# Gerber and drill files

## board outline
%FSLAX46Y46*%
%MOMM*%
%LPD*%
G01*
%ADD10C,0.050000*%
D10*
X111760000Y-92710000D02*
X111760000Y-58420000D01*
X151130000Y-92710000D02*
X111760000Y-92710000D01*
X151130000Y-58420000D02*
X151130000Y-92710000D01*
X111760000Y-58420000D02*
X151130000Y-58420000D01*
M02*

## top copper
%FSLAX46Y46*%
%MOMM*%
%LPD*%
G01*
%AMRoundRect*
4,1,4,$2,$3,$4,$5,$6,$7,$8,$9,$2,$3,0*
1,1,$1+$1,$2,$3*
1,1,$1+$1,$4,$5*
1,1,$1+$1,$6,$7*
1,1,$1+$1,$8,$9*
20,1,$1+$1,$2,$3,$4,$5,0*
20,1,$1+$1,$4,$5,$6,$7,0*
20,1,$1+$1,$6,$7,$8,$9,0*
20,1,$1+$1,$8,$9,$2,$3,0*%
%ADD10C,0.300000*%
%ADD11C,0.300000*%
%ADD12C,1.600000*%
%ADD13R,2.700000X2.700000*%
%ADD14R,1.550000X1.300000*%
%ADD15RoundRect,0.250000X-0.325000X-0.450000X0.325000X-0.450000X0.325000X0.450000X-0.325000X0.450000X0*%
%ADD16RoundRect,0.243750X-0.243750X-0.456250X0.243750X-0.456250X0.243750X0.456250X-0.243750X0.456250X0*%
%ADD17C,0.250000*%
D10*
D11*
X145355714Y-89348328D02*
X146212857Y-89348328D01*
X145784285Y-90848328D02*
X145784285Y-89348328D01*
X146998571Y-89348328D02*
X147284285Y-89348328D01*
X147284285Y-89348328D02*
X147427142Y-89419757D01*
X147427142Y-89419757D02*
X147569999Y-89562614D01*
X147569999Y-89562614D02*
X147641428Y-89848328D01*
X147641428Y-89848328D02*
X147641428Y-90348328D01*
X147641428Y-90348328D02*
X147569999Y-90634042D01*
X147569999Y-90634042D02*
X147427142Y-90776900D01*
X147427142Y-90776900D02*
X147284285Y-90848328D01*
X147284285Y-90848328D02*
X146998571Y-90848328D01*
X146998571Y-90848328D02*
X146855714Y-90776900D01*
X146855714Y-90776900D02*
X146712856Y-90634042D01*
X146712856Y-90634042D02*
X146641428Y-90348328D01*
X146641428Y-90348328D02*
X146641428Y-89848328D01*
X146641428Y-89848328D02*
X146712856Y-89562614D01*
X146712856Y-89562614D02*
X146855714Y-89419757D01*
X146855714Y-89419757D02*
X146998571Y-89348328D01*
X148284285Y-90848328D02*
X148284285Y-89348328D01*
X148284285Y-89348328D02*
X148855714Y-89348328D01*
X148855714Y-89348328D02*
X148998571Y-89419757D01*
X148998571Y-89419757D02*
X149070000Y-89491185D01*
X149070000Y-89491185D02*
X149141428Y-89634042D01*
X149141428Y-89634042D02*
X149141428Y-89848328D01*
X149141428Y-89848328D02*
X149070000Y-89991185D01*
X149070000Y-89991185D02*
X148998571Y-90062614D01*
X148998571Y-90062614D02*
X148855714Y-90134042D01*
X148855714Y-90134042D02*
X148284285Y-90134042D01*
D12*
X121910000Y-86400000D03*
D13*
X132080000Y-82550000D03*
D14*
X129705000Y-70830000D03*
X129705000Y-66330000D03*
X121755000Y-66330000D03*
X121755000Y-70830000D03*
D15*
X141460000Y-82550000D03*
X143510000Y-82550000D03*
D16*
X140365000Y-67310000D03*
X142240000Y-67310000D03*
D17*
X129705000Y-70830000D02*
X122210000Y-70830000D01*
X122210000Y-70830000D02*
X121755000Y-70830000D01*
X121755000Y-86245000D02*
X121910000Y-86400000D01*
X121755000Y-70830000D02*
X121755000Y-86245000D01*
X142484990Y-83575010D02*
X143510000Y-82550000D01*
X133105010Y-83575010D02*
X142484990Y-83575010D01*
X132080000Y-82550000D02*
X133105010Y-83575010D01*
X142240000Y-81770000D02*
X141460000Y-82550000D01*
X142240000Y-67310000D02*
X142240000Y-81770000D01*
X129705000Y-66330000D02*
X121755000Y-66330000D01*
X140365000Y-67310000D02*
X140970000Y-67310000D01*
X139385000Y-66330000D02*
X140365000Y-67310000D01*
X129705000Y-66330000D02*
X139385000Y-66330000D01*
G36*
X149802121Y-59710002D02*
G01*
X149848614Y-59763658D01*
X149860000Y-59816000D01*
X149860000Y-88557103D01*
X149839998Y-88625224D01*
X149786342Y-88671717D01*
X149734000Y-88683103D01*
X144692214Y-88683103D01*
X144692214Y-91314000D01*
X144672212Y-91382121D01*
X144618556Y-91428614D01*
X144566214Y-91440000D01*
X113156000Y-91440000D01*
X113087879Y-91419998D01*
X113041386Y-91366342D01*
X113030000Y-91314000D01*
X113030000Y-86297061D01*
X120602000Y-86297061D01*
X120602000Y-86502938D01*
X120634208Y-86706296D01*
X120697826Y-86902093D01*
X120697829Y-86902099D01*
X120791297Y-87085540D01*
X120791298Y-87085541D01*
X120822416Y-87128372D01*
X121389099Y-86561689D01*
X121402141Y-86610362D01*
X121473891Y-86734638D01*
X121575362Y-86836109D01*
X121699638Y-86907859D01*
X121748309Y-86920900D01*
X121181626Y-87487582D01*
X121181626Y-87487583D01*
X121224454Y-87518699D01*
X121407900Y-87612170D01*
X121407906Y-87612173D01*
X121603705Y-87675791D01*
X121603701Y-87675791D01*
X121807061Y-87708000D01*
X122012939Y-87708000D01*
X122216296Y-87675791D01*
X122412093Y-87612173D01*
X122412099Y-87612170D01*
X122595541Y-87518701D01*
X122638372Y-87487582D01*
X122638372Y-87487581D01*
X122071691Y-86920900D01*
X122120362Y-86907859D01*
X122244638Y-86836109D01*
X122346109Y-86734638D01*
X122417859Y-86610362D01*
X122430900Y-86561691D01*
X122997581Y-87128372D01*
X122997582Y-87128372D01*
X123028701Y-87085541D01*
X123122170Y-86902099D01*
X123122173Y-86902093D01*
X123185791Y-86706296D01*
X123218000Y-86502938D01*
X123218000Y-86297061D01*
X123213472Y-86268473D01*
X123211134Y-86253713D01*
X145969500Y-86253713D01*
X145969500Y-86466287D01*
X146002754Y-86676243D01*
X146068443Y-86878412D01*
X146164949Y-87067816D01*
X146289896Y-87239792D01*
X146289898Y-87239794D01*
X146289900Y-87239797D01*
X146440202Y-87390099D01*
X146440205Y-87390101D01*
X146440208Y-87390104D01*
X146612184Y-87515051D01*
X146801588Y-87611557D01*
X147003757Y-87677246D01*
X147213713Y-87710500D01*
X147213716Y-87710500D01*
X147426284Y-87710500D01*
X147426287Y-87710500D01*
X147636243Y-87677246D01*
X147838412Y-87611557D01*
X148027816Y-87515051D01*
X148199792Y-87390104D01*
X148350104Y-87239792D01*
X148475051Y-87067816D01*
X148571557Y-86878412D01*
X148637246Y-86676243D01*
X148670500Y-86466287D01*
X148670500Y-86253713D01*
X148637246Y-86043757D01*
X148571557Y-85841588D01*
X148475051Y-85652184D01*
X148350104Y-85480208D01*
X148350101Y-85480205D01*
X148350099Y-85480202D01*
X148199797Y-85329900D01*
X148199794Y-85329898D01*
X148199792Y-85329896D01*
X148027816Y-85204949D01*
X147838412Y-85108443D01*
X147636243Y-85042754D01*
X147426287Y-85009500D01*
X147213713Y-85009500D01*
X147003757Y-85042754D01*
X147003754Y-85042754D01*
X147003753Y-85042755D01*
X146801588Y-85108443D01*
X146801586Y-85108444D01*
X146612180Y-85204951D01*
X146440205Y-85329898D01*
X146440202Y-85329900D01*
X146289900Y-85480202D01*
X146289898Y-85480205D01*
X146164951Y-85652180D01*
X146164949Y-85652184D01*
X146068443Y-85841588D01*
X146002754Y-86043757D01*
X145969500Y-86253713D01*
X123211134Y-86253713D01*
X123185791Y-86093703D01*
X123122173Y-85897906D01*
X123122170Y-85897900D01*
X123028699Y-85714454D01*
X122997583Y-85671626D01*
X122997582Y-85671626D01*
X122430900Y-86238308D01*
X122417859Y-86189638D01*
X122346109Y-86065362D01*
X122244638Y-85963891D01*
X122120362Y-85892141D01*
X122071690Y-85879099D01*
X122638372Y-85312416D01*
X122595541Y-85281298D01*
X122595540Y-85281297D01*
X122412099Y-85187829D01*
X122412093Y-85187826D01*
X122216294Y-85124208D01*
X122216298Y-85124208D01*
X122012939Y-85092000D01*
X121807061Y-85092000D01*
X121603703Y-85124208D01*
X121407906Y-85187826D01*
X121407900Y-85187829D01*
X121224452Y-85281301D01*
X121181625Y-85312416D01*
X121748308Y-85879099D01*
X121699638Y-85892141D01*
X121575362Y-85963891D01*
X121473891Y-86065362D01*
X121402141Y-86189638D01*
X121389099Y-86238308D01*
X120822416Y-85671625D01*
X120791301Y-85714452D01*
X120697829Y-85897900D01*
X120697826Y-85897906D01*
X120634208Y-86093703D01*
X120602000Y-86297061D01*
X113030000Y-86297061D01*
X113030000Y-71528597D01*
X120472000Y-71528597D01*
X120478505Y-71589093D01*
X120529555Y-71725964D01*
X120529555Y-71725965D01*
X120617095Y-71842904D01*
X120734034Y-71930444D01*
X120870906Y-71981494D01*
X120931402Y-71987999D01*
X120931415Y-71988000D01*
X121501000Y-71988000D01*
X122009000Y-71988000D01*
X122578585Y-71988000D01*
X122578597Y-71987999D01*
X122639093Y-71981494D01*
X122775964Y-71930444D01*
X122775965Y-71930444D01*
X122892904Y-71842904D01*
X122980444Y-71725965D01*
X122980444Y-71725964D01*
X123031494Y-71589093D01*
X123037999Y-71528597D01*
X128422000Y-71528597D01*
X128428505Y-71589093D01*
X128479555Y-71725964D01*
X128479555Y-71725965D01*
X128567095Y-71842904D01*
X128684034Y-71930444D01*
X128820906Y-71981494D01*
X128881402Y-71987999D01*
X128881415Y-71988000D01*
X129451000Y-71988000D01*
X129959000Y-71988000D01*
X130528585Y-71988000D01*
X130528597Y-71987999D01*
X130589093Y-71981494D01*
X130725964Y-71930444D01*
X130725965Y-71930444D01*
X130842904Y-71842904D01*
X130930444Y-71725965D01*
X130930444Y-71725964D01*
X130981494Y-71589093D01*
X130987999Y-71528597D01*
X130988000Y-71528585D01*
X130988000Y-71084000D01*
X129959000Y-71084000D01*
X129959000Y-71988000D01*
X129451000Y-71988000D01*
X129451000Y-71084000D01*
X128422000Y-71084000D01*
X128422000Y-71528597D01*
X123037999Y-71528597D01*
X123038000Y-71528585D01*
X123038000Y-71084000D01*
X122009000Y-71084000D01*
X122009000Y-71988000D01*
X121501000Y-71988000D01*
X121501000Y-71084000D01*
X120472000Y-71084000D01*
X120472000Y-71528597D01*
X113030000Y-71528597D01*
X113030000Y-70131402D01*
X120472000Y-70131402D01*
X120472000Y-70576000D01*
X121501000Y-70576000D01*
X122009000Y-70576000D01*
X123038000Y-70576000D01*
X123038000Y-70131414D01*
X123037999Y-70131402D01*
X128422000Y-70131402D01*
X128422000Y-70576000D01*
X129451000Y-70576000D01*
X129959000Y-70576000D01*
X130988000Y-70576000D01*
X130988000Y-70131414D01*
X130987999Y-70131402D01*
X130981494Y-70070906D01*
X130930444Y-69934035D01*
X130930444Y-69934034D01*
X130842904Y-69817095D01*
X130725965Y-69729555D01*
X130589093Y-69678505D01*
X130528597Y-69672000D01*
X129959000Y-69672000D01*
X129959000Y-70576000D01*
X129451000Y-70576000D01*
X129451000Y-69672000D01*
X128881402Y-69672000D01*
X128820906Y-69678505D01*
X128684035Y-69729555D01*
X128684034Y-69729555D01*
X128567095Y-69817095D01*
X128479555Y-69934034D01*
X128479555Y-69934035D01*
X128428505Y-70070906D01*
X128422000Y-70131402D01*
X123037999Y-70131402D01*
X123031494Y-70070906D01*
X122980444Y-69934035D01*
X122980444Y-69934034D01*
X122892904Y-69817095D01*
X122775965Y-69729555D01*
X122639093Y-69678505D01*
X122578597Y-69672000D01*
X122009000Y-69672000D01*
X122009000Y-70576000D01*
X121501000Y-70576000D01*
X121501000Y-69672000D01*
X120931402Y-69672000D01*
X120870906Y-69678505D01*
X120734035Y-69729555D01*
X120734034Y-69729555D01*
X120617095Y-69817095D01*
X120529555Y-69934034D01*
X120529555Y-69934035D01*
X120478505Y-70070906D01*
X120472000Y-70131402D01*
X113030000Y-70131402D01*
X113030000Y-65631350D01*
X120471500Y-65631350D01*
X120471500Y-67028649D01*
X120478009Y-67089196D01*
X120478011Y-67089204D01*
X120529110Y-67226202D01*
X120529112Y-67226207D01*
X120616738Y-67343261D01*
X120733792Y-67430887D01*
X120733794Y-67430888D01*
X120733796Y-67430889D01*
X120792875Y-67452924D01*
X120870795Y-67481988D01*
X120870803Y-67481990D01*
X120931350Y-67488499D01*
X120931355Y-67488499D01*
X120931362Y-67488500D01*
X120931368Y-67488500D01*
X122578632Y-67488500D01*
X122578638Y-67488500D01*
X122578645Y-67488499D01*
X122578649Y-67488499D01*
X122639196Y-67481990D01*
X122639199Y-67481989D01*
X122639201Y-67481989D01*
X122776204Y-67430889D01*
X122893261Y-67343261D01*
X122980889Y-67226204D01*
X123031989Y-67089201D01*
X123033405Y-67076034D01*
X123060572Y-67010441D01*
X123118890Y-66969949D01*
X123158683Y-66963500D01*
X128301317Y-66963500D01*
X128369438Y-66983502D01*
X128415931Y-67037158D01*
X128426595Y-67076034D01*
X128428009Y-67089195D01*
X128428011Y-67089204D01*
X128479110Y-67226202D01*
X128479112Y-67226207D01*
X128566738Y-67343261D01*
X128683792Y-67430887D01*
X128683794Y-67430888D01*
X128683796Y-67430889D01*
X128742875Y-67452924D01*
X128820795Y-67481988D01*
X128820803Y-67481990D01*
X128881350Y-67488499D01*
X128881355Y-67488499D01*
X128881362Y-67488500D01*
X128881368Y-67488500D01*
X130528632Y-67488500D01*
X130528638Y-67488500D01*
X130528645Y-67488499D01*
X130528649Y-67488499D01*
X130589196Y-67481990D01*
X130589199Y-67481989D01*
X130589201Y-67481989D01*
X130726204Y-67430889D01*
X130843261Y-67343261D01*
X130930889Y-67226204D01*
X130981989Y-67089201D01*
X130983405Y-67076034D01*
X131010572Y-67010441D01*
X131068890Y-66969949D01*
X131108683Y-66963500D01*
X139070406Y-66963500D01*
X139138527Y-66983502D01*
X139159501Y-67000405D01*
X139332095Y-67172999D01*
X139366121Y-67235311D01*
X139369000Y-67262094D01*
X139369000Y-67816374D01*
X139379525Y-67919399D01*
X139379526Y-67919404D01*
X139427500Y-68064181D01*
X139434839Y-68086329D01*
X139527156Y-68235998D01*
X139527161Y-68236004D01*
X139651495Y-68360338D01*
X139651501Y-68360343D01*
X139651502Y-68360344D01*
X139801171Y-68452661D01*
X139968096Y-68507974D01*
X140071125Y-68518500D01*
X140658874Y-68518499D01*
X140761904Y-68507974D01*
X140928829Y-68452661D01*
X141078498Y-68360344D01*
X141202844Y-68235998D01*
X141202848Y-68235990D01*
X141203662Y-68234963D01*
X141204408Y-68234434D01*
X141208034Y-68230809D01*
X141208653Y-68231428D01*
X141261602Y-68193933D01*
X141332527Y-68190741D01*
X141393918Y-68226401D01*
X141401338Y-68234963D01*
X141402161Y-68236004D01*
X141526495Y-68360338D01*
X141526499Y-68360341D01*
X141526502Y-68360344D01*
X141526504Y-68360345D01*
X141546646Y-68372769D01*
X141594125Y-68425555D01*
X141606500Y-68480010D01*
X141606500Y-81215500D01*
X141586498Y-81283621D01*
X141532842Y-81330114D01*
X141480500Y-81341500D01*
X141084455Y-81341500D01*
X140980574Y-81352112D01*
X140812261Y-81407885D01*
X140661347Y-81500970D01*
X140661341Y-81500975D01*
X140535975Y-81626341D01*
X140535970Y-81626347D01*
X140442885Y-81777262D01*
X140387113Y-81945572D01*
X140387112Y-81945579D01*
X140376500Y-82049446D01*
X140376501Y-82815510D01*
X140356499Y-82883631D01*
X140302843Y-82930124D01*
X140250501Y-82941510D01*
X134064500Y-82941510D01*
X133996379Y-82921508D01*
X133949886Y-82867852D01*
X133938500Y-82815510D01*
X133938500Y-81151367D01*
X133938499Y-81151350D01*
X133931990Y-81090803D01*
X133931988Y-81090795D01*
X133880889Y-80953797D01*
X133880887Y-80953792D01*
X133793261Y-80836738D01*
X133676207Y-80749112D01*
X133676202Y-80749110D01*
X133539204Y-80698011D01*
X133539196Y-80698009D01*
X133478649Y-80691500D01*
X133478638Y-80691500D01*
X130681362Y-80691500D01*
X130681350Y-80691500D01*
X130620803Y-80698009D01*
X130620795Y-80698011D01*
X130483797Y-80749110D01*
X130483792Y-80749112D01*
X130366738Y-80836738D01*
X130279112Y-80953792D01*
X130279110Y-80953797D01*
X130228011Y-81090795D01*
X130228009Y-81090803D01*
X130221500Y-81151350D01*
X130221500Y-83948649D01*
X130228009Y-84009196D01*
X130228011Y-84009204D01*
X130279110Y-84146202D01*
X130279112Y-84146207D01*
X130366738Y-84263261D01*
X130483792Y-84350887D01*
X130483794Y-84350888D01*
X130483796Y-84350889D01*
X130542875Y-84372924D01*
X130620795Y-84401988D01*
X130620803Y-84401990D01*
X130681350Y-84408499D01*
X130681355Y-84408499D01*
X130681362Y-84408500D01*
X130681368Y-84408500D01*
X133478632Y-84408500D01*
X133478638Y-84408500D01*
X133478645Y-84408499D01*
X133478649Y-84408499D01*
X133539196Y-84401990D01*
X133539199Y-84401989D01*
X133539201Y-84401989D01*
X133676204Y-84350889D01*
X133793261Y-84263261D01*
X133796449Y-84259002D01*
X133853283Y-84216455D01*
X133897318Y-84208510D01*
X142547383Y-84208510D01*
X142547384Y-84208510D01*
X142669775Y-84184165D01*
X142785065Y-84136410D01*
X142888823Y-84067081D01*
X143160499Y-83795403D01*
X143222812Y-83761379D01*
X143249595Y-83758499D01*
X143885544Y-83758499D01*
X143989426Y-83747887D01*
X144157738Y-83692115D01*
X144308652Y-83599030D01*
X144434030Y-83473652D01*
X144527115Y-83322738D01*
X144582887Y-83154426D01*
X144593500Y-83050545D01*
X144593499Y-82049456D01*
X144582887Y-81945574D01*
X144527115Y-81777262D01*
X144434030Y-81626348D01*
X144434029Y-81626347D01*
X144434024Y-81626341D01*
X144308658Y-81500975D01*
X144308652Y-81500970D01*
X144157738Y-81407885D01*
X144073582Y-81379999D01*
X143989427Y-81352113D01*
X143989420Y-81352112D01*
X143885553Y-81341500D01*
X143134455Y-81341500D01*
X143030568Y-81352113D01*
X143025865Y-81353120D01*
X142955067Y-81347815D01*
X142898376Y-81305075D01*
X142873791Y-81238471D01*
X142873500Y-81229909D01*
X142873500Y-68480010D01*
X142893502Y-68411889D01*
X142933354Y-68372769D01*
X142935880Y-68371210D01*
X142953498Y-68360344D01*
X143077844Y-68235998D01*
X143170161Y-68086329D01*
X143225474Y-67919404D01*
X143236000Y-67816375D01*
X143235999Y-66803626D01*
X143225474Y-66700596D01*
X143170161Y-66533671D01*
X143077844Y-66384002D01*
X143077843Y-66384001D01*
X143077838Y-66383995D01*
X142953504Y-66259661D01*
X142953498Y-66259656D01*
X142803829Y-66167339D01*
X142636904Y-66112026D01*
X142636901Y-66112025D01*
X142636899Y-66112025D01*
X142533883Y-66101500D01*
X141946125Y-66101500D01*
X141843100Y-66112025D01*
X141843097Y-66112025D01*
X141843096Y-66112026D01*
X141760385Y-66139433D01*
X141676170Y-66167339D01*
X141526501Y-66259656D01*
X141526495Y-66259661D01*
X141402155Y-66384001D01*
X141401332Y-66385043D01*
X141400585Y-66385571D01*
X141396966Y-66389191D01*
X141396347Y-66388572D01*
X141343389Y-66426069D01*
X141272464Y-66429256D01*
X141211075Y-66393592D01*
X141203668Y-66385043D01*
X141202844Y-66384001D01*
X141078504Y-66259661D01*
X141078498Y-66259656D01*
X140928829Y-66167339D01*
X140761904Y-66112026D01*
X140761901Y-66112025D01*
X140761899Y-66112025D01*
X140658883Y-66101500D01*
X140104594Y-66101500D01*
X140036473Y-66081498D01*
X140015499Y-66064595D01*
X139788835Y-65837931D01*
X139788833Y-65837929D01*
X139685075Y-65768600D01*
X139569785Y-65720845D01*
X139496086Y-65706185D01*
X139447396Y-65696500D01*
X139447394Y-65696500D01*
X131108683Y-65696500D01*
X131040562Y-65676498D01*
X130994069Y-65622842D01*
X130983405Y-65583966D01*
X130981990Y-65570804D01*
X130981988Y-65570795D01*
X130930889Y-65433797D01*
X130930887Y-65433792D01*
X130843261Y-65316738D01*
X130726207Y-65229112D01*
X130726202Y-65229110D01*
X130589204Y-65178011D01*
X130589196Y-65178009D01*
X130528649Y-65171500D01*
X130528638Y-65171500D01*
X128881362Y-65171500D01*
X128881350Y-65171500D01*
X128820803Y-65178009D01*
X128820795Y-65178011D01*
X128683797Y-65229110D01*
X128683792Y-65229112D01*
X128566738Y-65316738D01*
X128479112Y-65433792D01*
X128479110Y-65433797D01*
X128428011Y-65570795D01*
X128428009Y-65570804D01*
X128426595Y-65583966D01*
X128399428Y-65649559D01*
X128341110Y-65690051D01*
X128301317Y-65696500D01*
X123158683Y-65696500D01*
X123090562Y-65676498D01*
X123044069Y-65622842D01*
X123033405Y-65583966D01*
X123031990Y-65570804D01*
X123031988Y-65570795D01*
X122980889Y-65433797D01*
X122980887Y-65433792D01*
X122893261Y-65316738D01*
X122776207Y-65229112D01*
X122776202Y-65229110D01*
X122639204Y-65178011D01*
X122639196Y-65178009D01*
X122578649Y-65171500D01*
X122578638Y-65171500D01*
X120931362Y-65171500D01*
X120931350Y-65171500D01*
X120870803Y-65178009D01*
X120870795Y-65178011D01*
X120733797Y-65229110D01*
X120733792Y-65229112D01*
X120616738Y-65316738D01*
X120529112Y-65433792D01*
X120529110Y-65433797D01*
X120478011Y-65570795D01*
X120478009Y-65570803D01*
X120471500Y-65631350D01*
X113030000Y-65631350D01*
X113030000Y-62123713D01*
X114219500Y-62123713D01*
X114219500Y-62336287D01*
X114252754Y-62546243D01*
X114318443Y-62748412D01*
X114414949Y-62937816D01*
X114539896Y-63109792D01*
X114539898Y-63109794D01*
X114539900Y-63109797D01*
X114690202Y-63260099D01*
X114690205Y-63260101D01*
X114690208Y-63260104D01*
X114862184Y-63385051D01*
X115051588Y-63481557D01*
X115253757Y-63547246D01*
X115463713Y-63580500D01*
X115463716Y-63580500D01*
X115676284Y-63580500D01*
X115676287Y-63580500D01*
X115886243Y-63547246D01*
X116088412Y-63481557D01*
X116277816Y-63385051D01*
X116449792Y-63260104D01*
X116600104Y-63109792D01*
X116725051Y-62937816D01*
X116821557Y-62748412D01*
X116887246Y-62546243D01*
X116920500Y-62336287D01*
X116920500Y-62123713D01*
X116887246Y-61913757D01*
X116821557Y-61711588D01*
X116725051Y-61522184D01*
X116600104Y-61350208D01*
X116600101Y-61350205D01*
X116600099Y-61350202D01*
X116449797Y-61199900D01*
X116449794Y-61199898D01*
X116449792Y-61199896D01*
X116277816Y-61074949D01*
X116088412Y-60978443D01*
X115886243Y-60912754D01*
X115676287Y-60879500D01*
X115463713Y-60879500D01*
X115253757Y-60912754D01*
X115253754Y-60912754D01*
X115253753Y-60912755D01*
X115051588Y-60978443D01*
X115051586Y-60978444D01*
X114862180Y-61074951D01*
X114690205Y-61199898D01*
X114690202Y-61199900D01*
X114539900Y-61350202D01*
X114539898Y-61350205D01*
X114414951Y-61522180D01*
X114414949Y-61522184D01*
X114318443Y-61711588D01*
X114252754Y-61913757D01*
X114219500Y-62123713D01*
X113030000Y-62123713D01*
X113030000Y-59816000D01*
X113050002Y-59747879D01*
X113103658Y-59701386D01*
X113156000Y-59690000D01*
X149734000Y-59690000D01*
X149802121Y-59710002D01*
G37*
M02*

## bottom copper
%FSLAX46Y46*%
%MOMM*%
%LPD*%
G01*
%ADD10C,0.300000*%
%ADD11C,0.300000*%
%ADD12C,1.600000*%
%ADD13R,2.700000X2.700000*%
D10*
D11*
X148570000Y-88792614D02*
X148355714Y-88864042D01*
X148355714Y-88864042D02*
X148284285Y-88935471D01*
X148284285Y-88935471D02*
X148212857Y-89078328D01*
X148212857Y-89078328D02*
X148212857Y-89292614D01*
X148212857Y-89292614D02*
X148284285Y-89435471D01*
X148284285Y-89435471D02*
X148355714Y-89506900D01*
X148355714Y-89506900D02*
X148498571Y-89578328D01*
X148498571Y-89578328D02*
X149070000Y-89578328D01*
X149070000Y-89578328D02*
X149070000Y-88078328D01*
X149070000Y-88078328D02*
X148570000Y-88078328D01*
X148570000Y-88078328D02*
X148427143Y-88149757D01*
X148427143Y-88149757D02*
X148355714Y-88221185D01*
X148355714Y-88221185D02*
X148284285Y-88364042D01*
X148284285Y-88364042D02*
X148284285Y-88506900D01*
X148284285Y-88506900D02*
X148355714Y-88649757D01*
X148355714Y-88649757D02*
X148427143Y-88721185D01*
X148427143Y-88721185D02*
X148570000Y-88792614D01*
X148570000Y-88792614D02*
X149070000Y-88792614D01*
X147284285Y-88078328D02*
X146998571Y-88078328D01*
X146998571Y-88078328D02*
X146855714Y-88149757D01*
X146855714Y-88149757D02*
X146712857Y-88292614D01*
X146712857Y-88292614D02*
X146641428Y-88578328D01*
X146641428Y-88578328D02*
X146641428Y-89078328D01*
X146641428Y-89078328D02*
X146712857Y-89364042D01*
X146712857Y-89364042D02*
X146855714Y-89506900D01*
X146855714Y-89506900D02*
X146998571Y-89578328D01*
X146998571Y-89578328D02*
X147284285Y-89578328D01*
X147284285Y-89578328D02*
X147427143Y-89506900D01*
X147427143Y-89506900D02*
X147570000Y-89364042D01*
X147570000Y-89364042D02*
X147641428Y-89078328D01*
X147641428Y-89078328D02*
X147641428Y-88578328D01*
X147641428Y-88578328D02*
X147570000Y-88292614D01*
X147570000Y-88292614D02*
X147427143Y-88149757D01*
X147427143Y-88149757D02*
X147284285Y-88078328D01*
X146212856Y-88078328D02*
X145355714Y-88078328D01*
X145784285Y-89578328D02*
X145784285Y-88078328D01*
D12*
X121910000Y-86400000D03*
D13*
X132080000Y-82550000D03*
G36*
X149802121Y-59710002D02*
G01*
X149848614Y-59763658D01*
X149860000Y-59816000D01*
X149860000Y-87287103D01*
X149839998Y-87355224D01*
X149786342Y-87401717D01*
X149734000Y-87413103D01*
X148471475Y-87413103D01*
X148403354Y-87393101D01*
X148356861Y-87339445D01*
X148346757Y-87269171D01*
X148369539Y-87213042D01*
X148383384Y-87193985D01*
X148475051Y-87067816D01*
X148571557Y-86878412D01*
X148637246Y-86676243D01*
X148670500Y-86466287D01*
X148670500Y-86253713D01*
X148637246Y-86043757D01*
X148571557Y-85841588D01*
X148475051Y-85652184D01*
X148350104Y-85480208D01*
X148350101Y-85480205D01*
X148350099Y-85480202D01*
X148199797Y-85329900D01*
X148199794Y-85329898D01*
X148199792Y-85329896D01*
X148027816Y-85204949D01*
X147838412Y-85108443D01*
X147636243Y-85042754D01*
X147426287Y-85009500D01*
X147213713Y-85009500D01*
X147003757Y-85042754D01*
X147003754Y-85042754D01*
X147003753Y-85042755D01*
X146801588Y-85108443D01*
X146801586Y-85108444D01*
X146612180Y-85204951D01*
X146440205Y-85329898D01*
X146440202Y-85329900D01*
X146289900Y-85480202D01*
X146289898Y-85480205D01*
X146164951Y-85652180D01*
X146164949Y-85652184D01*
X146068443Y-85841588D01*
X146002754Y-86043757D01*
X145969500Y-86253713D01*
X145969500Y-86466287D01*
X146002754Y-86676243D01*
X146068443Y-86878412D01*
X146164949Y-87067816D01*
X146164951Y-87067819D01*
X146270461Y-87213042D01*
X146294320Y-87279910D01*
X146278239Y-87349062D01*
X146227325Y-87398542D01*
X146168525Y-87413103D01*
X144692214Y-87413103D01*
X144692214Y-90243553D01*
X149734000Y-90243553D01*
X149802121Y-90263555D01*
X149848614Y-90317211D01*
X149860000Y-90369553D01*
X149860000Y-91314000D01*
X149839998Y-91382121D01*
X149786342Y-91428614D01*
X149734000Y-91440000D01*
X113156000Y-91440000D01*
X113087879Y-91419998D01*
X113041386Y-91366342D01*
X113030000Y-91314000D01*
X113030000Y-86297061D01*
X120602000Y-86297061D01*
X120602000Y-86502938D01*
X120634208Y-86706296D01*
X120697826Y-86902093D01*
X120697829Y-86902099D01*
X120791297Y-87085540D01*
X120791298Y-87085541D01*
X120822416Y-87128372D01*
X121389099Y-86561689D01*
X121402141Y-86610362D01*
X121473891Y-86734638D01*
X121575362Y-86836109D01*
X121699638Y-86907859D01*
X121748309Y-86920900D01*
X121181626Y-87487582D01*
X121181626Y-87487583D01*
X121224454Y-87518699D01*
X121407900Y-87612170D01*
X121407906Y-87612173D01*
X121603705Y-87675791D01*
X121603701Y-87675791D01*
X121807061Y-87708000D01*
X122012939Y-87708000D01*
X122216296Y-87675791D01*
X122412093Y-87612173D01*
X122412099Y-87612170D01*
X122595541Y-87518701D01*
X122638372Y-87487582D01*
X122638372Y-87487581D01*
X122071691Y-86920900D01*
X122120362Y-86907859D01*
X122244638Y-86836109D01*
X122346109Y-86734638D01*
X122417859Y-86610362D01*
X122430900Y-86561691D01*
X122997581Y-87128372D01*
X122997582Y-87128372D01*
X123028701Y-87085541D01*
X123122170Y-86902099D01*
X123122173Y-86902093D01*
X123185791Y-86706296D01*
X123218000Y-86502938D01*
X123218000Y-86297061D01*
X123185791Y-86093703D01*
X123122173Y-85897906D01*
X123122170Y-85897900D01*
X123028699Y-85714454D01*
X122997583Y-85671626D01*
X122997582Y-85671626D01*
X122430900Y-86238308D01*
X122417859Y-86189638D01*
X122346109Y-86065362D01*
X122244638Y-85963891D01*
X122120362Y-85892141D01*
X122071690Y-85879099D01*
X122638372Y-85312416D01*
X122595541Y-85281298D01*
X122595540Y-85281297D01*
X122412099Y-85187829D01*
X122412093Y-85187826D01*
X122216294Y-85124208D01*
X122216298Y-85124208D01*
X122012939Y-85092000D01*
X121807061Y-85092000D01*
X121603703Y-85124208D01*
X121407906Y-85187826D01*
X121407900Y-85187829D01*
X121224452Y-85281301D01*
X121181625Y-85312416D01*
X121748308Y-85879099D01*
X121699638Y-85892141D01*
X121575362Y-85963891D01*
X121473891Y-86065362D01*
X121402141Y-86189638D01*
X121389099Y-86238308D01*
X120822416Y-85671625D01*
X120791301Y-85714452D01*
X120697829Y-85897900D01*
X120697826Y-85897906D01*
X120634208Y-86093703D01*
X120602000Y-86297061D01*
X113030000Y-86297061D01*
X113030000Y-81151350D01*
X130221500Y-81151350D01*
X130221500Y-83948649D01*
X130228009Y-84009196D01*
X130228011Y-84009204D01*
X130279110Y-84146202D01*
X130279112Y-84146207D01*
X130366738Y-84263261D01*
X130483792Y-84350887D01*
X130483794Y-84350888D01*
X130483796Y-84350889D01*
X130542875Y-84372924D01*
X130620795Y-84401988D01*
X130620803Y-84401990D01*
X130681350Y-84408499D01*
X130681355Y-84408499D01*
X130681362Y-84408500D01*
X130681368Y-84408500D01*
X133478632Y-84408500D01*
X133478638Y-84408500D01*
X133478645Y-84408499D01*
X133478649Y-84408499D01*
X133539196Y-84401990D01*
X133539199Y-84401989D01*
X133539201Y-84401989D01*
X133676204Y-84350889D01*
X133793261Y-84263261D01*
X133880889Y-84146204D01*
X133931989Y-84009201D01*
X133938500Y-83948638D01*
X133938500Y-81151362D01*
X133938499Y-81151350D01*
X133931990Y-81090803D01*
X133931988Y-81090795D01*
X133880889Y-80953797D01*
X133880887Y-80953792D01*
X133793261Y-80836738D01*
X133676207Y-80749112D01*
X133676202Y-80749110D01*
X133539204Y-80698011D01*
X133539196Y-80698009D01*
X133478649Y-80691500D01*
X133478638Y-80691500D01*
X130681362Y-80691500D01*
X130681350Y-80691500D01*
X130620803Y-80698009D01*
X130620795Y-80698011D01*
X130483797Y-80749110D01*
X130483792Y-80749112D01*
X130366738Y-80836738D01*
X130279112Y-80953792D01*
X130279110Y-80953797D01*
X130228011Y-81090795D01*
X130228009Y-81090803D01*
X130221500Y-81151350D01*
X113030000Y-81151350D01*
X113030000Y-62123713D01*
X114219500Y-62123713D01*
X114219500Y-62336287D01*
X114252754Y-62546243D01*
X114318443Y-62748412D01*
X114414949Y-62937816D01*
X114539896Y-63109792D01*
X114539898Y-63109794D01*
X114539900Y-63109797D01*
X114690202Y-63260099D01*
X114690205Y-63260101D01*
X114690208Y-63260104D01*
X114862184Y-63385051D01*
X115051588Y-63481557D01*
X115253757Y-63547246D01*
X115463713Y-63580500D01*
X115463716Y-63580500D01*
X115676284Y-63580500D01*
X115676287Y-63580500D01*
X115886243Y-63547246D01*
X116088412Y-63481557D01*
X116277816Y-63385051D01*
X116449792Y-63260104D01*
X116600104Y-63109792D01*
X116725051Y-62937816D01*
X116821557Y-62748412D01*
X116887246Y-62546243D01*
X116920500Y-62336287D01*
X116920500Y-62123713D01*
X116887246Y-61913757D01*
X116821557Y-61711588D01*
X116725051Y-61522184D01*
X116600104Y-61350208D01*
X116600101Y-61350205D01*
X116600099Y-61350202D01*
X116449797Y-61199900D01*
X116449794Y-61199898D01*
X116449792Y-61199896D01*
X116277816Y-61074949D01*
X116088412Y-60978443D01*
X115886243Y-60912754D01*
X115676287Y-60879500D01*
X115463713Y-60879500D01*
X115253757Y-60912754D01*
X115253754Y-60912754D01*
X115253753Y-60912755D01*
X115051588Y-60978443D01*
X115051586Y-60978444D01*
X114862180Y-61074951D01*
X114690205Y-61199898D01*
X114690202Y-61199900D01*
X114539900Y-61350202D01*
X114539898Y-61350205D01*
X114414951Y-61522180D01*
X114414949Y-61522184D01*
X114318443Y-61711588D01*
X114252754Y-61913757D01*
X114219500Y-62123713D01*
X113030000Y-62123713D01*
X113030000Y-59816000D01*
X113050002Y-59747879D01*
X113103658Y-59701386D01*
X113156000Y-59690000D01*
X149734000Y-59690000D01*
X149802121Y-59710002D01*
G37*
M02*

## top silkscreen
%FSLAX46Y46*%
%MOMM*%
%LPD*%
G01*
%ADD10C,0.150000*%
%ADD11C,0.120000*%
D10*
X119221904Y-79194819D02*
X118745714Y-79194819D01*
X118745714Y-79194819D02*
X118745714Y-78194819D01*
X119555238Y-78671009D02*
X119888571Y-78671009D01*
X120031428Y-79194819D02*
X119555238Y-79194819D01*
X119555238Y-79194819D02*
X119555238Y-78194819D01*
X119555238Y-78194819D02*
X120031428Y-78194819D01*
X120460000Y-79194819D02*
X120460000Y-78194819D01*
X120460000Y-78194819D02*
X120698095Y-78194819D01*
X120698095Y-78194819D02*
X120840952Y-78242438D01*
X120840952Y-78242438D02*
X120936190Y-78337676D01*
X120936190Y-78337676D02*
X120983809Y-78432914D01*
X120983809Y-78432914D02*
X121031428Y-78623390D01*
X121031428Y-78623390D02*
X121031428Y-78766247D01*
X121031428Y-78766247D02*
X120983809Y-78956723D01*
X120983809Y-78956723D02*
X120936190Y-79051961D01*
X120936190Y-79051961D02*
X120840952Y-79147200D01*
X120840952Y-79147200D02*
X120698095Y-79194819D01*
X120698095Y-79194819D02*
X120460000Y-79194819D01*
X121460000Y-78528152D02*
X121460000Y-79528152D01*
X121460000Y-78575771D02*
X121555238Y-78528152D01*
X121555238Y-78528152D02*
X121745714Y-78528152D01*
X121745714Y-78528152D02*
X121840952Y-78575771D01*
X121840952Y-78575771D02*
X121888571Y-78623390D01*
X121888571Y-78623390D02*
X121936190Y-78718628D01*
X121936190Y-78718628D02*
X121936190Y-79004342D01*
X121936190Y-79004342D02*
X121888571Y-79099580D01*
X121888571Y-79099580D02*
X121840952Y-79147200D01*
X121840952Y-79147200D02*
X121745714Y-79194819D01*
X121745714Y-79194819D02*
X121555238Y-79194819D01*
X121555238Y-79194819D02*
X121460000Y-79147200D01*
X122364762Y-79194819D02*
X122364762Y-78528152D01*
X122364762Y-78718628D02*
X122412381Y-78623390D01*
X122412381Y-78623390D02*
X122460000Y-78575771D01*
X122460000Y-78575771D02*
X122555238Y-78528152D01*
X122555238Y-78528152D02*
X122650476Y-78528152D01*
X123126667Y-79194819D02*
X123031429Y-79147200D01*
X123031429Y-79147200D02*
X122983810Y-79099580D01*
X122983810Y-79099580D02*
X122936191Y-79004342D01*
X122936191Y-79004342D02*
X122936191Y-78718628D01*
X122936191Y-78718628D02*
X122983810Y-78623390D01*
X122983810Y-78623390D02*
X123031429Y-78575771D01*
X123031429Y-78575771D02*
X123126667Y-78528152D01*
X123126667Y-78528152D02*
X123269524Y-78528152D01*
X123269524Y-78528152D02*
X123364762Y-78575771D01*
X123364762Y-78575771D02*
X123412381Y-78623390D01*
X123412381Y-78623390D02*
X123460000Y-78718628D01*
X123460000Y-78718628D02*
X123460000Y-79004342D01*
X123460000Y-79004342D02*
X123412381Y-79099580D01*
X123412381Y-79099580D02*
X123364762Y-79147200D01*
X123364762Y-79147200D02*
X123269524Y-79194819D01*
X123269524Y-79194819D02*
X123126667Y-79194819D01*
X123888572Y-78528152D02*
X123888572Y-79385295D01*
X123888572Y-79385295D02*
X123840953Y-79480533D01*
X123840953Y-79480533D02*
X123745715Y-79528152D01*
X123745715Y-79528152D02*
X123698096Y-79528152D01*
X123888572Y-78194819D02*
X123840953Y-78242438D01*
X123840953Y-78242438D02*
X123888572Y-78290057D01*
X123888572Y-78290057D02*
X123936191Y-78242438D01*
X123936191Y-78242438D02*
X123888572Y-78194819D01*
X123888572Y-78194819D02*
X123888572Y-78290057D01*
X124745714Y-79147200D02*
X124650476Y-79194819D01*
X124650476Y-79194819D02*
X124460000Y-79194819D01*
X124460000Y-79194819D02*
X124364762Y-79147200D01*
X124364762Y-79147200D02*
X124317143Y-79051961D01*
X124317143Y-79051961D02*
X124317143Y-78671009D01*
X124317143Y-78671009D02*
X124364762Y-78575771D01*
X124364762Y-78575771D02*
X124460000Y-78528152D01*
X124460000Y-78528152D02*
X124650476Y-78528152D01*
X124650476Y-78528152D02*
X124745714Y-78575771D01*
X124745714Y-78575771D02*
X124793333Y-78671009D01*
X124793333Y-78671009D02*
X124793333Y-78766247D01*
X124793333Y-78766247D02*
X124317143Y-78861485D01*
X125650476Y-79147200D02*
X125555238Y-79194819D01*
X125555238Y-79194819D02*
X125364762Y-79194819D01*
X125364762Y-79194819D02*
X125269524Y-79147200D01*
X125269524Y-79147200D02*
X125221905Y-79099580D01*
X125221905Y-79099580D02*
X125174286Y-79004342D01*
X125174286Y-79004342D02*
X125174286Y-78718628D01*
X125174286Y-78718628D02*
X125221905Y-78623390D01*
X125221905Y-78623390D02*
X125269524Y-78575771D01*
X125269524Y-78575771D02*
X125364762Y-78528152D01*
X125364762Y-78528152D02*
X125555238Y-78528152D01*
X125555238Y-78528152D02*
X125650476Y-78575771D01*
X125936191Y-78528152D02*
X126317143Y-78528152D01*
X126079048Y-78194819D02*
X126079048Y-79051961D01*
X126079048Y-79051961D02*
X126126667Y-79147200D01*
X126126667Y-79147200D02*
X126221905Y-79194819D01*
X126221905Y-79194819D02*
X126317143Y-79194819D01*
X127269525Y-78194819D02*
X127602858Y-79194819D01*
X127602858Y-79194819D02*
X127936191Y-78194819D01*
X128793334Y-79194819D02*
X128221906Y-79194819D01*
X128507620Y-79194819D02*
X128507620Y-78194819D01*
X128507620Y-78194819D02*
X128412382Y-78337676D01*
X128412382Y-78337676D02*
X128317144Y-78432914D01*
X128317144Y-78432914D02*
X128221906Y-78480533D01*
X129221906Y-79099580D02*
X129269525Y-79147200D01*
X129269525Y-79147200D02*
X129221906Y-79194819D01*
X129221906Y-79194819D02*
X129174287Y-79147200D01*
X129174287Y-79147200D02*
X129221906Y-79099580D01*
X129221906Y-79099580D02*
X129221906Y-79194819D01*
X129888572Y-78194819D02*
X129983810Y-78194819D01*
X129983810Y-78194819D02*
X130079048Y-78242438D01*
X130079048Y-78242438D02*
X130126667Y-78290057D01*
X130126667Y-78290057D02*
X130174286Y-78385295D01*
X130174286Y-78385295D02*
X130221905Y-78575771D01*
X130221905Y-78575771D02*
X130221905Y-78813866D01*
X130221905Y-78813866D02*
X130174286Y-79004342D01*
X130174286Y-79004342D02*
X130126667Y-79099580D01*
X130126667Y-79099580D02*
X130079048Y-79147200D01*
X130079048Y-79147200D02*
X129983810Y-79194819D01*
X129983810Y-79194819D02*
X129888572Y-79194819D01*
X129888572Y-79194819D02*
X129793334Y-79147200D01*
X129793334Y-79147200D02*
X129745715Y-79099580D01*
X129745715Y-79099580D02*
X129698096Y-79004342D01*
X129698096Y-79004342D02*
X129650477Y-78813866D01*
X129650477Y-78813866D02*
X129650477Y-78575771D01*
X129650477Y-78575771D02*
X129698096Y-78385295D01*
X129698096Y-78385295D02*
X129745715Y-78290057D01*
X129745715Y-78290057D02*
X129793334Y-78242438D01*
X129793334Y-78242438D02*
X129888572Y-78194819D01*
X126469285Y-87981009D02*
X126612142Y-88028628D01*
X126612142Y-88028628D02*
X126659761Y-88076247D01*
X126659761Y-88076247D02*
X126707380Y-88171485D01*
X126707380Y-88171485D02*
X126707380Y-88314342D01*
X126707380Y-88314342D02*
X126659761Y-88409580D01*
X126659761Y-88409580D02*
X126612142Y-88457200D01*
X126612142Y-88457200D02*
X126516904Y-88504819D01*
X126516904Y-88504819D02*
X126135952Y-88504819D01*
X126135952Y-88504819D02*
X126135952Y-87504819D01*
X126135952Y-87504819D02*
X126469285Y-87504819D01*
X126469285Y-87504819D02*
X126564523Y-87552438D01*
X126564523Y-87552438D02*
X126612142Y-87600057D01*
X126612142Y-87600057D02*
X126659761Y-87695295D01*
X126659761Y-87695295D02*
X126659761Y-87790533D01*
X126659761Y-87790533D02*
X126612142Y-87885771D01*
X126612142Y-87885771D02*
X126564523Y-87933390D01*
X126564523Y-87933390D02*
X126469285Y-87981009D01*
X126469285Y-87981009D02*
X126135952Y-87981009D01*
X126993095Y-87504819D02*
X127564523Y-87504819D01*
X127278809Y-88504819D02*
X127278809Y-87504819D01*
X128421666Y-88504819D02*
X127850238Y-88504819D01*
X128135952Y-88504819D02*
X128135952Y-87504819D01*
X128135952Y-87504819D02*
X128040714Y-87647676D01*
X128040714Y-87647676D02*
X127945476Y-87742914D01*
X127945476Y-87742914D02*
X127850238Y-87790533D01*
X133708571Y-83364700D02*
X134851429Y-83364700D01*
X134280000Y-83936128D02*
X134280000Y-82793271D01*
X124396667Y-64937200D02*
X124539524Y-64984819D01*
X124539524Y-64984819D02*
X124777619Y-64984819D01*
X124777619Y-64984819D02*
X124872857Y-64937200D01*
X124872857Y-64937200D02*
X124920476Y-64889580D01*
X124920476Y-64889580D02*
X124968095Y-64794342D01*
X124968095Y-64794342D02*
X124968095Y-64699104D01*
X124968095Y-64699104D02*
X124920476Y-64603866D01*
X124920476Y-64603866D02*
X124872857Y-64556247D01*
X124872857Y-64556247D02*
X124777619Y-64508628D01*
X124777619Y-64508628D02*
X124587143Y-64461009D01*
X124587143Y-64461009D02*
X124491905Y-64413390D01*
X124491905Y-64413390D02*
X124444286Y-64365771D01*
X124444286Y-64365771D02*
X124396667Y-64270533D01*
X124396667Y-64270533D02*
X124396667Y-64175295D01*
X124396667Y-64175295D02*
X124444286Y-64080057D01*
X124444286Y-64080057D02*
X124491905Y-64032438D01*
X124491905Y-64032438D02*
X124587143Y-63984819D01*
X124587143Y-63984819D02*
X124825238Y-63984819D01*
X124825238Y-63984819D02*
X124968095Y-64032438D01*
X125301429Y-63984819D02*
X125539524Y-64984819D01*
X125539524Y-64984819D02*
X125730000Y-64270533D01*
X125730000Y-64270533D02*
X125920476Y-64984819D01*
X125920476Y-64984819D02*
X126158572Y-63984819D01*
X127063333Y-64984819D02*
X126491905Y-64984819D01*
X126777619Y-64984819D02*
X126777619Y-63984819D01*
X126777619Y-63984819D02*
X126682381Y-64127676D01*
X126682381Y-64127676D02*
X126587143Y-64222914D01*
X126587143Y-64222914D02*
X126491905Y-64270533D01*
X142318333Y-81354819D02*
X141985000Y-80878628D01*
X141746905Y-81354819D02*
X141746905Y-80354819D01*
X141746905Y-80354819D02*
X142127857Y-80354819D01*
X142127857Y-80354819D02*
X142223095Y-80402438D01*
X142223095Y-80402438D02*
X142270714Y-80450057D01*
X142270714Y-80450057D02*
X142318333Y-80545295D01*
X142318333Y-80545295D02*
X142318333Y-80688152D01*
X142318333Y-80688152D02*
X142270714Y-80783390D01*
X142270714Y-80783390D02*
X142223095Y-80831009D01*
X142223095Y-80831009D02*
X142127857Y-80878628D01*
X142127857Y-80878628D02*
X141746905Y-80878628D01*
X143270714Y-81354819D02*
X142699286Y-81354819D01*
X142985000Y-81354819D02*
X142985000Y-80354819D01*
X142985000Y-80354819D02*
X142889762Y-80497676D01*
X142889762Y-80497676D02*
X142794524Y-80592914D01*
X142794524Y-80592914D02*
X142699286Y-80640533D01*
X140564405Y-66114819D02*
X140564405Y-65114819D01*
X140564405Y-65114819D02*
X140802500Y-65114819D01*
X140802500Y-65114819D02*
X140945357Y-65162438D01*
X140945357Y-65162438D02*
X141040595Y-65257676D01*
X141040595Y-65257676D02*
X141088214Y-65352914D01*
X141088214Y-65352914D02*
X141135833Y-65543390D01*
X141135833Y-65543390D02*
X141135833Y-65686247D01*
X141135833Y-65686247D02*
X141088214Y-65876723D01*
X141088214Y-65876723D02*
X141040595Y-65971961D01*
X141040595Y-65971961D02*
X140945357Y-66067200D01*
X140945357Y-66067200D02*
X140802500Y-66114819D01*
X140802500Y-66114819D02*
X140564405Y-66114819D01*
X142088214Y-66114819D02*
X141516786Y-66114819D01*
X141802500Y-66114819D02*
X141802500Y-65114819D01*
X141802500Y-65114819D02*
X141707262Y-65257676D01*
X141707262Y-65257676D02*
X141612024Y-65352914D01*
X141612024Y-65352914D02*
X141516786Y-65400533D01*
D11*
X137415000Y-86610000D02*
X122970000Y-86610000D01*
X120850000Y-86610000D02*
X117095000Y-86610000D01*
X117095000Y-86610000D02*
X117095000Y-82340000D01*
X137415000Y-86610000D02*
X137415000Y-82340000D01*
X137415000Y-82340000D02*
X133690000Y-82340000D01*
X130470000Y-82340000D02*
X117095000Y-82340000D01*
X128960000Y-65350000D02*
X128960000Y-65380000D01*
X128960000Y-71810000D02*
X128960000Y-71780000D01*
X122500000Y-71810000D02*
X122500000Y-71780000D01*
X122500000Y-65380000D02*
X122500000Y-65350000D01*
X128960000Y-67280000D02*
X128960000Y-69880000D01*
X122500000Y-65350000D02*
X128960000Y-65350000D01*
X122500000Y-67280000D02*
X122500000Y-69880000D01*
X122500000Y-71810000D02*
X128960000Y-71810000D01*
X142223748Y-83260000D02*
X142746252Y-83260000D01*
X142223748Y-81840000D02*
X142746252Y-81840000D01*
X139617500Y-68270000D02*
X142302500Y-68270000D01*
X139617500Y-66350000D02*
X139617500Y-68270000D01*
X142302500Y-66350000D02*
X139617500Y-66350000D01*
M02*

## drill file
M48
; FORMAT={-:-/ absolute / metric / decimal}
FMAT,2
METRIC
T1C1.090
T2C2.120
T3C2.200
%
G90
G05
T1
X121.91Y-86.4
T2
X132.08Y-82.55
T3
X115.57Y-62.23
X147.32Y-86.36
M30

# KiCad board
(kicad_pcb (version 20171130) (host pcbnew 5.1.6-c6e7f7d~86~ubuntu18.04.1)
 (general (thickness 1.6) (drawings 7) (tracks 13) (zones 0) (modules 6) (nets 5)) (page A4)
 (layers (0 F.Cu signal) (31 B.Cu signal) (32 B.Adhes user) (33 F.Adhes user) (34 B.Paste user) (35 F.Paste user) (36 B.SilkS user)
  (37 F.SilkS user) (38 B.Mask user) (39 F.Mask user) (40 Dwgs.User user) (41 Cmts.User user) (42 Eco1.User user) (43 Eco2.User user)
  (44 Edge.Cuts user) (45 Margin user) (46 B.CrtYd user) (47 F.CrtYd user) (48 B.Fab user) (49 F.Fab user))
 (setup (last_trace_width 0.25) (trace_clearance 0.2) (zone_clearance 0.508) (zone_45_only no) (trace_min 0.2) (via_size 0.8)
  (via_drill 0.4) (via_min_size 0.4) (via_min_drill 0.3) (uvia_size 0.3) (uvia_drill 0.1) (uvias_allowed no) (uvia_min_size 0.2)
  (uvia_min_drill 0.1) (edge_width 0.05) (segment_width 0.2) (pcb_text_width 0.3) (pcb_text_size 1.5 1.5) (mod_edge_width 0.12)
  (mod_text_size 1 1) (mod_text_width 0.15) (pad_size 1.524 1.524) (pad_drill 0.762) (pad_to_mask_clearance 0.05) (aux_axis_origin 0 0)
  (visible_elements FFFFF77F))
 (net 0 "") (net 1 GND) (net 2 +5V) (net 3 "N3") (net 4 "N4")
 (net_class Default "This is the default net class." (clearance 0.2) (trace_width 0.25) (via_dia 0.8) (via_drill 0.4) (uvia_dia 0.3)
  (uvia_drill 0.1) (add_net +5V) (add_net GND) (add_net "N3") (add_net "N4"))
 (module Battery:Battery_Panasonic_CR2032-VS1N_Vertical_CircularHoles (layer F.Cu) (at 132.08 82.55 180)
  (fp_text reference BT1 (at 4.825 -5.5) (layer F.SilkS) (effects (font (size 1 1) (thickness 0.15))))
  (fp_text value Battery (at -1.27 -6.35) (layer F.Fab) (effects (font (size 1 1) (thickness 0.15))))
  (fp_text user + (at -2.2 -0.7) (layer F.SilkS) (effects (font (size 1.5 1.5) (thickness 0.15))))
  (fp_line (start -5.335 -4.06) (end 9.11 -4.06) (layer F.SilkS) (width 0.12))
  (fp_line (start 11.23 -4.06) (end 14.985 -4.06) (layer F.SilkS) (width 0.12))
  (fp_line (start 14.985 -4.06) (end 14.985 0.21) (layer F.SilkS) (width 0.12))
  (fp_line (start -5.335 -4.06) (end -5.335 0.21) (layer F.SilkS) (width 0.12))
  (fp_line (start -5.335 0.21) (end -1.61 0.21) (layer F.SilkS) (width 0.12))
  (fp_line (start 1.61 0.21) (end 14.985 0.21) (layer F.SilkS) (width 0.12))
  (pad 2 thru_hole circle (at 10.17 -3.85 180) (size 1.6 1.6) (drill 1.09) (layers *.Cu *.Mask) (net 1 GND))
  (pad 1 thru_hole rect (at 0 0 270) (size 2.7 2.7) (drill 2.12) (layers *.Cu *.Mask) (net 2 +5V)))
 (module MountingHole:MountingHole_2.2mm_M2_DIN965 (layer F.Cu) (at 147.32 86.36)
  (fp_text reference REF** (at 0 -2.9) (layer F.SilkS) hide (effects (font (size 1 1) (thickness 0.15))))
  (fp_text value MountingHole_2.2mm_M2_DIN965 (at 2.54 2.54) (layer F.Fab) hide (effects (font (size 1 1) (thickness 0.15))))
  (pad 1 np_thru_hole circle (at 0 0) (size 2.2 2.2) (drill 2.2) (layers *.Cu *.Mask)))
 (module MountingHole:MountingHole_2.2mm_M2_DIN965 (layer F.Cu) (at 115.57 62.23)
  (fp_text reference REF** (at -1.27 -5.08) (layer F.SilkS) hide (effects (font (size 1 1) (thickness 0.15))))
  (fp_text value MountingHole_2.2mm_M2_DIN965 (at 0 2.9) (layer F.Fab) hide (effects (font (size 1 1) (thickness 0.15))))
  (pad 1 np_thru_hole circle (at 0 0) (size 2.2 2.2) (drill 2.2) (layers *.Cu *.Mask)))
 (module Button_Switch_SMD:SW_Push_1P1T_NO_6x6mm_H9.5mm (layer F.Cu) (at 125.73 68.58)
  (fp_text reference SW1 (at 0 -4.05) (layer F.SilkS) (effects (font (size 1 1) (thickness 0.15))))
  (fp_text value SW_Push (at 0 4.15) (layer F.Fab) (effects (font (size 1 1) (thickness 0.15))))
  (fp_line (start 3.23 -3.23) (end 3.23 -3.2) (layer F.SilkS) (width 0.12))
  (fp_line (start 3.23 3.23) (end 3.23 3.2) (layer F.SilkS) (width 0.12))
  (fp_line (start -3.23 3.23) (end -3.23 3.2) (layer F.SilkS) (width 0.12))
  (fp_line (start -3.23 -3.2) (end -3.23 -3.23) (layer F.SilkS) (width 0.12))
  (fp_line (start 3.23 -1.3) (end 3.23 1.3) (layer F.SilkS) (width 0.12))
  (fp_line (start -3.23 -3.23) (end 3.23 -3.23) (layer F.SilkS) (width 0.12))
  (fp_line (start -3.23 -1.3) (end -3.23 1.3) (layer F.SilkS) (width 0.12))
  (fp_line (start -3.23 3.23) (end 3.23 3.23) (layer F.SilkS) (width 0.12))
  (pad 2 smd rect (at 3.975 2.25) (size 1.55 1.3) (layers F.Cu F.Paste F.Mask) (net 1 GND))
  (pad 1 smd rect (at 3.975 -2.25) (size 1.55 1.3) (layers F.Cu F.Paste F.Mask) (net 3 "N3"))
  (pad 1 smd rect (at -3.975 -2.25) (size 1.55 1.3) (layers F.Cu F.Paste F.Mask) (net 3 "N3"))
  (pad 2 smd rect (at -3.975 2.25) (size 1.55 1.3) (layers F.Cu F.Paste F.Mask) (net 1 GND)))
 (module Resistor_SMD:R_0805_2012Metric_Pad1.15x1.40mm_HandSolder (layer F.Cu) (at 142.485 82.55)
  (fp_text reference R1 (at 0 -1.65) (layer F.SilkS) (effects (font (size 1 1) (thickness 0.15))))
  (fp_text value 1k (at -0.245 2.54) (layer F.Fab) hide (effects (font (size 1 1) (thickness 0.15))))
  (fp_line (start -0.261252 0.71) (end 0.261252 0.71) (layer F.SilkS) (width 0.12))
  (fp_line (start -0.261252 -0.71) (end 0.261252 -0.71) (layer F.SilkS) (width 0.12))
  (pad 1 smd roundrect (at -1.025 0) (size 1.15 1.4) (layers F.Cu F.Paste F.Mask) (roundrect_rratio 0.217391) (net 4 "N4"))
  (pad 2 smd roundrect (at 1.025 0) (size 1.15 1.4) (layers F.Cu F.Paste F.Mask) (roundrect_rratio 0.217391) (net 2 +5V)))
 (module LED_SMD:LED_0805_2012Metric (layer F.Cu) (at 141.3025 67.31)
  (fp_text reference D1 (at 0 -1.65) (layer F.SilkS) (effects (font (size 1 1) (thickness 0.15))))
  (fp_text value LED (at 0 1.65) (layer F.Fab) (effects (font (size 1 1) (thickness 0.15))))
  (fp_line (start -1.685 0.96) (end 1 0.96) (layer F.SilkS) (width 0.12))
  (fp_line (start -1.685 -0.96) (end -1.685 0.96) (layer F.SilkS) (width 0.12))
  (fp_line (start 1 -0.96) (end -1.685 -0.96) (layer F.SilkS) (width 0.12))
  (pad 1 smd roundrect (at -0.9375 0) (size 0.975 1.4) (layers F.Cu F.Paste F.Mask) (roundrect_rratio 0.25) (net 3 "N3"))
  (pad 2 smd roundrect (at 0.9375 0) (size 0.975 1.4) (layers F.Cu F.Paste F.Mask) (roundrect_rratio 0.25) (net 4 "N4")))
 (gr_line (start 111.76 92.71) (end 111.76 58.42) (layer Edge.Cuts) (width 0.05))
 (gr_line (start 151.13 92.71) (end 111.76 92.71) (layer Edge.Cuts) (width 0.05))
 (gr_line (start 151.13 58.42) (end 151.13 92.71) (layer Edge.Cuts) (width 0.05))
 (gr_line (start 111.76 58.42) (end 151.13 58.42) (layer Edge.Cuts) (width 0.05))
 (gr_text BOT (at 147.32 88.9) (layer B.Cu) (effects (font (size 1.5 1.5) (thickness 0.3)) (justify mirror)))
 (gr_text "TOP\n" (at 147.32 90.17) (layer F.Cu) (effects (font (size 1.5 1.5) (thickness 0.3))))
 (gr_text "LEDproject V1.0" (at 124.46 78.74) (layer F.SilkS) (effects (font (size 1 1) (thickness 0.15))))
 (segment (start 129.705 70.83) (end 122.21 70.83) (width 0.25) (layer F.Cu) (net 1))
 (segment (start 122.21 70.83) (end 121.755 70.83) (width 0.25) (layer F.Cu) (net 1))
 (segment (start 121.755 86.245) (end 121.91 86.4) (width 0.25) (layer F.Cu) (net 1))
 (segment (start 121.755 70.83) (end 121.755 86.245) (width 0.25) (layer F.Cu) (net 1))
 (segment (start 142.48499 83.57501) (end 143.51 82.55) (width 0.25) (layer F.Cu) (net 2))
 (segment (start 133.10501 83.57501) (end 142.48499 83.57501) (width 0.25) (layer F.Cu) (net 2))
 (segment (start 132.08 82.55) (end 133.10501 83.57501) (width 0.25) (layer F.Cu) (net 2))
 (segment (start 142.24 81.77) (end 141.46 82.55) (width 0.25) (layer F.Cu) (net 4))
 (segment (start 142.24 67.31) (end 142.24 81.77) (width 0.25) (layer F.Cu) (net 4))
 (segment (start 129.705 66.33) (end 121.755 66.33) (width 0.25) (layer F.Cu) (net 3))
 (segment (start 140.365 67.31) (end 140.97 67.31) (width 0.25) (layer F.Cu) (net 3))
 (segment (start 139.385 66.33) (end 140.365 67.31) (width 0.25) (layer F.Cu) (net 3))
 (segment (start 129.705 66.33) (end 139.385 66.33) (width 0.25) (layer F.Cu) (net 3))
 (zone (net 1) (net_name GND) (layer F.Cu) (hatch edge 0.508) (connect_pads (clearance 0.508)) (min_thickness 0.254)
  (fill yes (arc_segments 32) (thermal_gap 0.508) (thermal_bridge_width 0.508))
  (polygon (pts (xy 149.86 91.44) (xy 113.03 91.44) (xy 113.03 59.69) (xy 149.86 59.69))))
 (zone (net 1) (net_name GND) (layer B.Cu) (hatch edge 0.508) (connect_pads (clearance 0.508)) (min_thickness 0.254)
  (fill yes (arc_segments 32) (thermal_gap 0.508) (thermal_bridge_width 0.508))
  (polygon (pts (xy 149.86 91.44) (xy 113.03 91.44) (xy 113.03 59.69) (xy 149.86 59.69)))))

